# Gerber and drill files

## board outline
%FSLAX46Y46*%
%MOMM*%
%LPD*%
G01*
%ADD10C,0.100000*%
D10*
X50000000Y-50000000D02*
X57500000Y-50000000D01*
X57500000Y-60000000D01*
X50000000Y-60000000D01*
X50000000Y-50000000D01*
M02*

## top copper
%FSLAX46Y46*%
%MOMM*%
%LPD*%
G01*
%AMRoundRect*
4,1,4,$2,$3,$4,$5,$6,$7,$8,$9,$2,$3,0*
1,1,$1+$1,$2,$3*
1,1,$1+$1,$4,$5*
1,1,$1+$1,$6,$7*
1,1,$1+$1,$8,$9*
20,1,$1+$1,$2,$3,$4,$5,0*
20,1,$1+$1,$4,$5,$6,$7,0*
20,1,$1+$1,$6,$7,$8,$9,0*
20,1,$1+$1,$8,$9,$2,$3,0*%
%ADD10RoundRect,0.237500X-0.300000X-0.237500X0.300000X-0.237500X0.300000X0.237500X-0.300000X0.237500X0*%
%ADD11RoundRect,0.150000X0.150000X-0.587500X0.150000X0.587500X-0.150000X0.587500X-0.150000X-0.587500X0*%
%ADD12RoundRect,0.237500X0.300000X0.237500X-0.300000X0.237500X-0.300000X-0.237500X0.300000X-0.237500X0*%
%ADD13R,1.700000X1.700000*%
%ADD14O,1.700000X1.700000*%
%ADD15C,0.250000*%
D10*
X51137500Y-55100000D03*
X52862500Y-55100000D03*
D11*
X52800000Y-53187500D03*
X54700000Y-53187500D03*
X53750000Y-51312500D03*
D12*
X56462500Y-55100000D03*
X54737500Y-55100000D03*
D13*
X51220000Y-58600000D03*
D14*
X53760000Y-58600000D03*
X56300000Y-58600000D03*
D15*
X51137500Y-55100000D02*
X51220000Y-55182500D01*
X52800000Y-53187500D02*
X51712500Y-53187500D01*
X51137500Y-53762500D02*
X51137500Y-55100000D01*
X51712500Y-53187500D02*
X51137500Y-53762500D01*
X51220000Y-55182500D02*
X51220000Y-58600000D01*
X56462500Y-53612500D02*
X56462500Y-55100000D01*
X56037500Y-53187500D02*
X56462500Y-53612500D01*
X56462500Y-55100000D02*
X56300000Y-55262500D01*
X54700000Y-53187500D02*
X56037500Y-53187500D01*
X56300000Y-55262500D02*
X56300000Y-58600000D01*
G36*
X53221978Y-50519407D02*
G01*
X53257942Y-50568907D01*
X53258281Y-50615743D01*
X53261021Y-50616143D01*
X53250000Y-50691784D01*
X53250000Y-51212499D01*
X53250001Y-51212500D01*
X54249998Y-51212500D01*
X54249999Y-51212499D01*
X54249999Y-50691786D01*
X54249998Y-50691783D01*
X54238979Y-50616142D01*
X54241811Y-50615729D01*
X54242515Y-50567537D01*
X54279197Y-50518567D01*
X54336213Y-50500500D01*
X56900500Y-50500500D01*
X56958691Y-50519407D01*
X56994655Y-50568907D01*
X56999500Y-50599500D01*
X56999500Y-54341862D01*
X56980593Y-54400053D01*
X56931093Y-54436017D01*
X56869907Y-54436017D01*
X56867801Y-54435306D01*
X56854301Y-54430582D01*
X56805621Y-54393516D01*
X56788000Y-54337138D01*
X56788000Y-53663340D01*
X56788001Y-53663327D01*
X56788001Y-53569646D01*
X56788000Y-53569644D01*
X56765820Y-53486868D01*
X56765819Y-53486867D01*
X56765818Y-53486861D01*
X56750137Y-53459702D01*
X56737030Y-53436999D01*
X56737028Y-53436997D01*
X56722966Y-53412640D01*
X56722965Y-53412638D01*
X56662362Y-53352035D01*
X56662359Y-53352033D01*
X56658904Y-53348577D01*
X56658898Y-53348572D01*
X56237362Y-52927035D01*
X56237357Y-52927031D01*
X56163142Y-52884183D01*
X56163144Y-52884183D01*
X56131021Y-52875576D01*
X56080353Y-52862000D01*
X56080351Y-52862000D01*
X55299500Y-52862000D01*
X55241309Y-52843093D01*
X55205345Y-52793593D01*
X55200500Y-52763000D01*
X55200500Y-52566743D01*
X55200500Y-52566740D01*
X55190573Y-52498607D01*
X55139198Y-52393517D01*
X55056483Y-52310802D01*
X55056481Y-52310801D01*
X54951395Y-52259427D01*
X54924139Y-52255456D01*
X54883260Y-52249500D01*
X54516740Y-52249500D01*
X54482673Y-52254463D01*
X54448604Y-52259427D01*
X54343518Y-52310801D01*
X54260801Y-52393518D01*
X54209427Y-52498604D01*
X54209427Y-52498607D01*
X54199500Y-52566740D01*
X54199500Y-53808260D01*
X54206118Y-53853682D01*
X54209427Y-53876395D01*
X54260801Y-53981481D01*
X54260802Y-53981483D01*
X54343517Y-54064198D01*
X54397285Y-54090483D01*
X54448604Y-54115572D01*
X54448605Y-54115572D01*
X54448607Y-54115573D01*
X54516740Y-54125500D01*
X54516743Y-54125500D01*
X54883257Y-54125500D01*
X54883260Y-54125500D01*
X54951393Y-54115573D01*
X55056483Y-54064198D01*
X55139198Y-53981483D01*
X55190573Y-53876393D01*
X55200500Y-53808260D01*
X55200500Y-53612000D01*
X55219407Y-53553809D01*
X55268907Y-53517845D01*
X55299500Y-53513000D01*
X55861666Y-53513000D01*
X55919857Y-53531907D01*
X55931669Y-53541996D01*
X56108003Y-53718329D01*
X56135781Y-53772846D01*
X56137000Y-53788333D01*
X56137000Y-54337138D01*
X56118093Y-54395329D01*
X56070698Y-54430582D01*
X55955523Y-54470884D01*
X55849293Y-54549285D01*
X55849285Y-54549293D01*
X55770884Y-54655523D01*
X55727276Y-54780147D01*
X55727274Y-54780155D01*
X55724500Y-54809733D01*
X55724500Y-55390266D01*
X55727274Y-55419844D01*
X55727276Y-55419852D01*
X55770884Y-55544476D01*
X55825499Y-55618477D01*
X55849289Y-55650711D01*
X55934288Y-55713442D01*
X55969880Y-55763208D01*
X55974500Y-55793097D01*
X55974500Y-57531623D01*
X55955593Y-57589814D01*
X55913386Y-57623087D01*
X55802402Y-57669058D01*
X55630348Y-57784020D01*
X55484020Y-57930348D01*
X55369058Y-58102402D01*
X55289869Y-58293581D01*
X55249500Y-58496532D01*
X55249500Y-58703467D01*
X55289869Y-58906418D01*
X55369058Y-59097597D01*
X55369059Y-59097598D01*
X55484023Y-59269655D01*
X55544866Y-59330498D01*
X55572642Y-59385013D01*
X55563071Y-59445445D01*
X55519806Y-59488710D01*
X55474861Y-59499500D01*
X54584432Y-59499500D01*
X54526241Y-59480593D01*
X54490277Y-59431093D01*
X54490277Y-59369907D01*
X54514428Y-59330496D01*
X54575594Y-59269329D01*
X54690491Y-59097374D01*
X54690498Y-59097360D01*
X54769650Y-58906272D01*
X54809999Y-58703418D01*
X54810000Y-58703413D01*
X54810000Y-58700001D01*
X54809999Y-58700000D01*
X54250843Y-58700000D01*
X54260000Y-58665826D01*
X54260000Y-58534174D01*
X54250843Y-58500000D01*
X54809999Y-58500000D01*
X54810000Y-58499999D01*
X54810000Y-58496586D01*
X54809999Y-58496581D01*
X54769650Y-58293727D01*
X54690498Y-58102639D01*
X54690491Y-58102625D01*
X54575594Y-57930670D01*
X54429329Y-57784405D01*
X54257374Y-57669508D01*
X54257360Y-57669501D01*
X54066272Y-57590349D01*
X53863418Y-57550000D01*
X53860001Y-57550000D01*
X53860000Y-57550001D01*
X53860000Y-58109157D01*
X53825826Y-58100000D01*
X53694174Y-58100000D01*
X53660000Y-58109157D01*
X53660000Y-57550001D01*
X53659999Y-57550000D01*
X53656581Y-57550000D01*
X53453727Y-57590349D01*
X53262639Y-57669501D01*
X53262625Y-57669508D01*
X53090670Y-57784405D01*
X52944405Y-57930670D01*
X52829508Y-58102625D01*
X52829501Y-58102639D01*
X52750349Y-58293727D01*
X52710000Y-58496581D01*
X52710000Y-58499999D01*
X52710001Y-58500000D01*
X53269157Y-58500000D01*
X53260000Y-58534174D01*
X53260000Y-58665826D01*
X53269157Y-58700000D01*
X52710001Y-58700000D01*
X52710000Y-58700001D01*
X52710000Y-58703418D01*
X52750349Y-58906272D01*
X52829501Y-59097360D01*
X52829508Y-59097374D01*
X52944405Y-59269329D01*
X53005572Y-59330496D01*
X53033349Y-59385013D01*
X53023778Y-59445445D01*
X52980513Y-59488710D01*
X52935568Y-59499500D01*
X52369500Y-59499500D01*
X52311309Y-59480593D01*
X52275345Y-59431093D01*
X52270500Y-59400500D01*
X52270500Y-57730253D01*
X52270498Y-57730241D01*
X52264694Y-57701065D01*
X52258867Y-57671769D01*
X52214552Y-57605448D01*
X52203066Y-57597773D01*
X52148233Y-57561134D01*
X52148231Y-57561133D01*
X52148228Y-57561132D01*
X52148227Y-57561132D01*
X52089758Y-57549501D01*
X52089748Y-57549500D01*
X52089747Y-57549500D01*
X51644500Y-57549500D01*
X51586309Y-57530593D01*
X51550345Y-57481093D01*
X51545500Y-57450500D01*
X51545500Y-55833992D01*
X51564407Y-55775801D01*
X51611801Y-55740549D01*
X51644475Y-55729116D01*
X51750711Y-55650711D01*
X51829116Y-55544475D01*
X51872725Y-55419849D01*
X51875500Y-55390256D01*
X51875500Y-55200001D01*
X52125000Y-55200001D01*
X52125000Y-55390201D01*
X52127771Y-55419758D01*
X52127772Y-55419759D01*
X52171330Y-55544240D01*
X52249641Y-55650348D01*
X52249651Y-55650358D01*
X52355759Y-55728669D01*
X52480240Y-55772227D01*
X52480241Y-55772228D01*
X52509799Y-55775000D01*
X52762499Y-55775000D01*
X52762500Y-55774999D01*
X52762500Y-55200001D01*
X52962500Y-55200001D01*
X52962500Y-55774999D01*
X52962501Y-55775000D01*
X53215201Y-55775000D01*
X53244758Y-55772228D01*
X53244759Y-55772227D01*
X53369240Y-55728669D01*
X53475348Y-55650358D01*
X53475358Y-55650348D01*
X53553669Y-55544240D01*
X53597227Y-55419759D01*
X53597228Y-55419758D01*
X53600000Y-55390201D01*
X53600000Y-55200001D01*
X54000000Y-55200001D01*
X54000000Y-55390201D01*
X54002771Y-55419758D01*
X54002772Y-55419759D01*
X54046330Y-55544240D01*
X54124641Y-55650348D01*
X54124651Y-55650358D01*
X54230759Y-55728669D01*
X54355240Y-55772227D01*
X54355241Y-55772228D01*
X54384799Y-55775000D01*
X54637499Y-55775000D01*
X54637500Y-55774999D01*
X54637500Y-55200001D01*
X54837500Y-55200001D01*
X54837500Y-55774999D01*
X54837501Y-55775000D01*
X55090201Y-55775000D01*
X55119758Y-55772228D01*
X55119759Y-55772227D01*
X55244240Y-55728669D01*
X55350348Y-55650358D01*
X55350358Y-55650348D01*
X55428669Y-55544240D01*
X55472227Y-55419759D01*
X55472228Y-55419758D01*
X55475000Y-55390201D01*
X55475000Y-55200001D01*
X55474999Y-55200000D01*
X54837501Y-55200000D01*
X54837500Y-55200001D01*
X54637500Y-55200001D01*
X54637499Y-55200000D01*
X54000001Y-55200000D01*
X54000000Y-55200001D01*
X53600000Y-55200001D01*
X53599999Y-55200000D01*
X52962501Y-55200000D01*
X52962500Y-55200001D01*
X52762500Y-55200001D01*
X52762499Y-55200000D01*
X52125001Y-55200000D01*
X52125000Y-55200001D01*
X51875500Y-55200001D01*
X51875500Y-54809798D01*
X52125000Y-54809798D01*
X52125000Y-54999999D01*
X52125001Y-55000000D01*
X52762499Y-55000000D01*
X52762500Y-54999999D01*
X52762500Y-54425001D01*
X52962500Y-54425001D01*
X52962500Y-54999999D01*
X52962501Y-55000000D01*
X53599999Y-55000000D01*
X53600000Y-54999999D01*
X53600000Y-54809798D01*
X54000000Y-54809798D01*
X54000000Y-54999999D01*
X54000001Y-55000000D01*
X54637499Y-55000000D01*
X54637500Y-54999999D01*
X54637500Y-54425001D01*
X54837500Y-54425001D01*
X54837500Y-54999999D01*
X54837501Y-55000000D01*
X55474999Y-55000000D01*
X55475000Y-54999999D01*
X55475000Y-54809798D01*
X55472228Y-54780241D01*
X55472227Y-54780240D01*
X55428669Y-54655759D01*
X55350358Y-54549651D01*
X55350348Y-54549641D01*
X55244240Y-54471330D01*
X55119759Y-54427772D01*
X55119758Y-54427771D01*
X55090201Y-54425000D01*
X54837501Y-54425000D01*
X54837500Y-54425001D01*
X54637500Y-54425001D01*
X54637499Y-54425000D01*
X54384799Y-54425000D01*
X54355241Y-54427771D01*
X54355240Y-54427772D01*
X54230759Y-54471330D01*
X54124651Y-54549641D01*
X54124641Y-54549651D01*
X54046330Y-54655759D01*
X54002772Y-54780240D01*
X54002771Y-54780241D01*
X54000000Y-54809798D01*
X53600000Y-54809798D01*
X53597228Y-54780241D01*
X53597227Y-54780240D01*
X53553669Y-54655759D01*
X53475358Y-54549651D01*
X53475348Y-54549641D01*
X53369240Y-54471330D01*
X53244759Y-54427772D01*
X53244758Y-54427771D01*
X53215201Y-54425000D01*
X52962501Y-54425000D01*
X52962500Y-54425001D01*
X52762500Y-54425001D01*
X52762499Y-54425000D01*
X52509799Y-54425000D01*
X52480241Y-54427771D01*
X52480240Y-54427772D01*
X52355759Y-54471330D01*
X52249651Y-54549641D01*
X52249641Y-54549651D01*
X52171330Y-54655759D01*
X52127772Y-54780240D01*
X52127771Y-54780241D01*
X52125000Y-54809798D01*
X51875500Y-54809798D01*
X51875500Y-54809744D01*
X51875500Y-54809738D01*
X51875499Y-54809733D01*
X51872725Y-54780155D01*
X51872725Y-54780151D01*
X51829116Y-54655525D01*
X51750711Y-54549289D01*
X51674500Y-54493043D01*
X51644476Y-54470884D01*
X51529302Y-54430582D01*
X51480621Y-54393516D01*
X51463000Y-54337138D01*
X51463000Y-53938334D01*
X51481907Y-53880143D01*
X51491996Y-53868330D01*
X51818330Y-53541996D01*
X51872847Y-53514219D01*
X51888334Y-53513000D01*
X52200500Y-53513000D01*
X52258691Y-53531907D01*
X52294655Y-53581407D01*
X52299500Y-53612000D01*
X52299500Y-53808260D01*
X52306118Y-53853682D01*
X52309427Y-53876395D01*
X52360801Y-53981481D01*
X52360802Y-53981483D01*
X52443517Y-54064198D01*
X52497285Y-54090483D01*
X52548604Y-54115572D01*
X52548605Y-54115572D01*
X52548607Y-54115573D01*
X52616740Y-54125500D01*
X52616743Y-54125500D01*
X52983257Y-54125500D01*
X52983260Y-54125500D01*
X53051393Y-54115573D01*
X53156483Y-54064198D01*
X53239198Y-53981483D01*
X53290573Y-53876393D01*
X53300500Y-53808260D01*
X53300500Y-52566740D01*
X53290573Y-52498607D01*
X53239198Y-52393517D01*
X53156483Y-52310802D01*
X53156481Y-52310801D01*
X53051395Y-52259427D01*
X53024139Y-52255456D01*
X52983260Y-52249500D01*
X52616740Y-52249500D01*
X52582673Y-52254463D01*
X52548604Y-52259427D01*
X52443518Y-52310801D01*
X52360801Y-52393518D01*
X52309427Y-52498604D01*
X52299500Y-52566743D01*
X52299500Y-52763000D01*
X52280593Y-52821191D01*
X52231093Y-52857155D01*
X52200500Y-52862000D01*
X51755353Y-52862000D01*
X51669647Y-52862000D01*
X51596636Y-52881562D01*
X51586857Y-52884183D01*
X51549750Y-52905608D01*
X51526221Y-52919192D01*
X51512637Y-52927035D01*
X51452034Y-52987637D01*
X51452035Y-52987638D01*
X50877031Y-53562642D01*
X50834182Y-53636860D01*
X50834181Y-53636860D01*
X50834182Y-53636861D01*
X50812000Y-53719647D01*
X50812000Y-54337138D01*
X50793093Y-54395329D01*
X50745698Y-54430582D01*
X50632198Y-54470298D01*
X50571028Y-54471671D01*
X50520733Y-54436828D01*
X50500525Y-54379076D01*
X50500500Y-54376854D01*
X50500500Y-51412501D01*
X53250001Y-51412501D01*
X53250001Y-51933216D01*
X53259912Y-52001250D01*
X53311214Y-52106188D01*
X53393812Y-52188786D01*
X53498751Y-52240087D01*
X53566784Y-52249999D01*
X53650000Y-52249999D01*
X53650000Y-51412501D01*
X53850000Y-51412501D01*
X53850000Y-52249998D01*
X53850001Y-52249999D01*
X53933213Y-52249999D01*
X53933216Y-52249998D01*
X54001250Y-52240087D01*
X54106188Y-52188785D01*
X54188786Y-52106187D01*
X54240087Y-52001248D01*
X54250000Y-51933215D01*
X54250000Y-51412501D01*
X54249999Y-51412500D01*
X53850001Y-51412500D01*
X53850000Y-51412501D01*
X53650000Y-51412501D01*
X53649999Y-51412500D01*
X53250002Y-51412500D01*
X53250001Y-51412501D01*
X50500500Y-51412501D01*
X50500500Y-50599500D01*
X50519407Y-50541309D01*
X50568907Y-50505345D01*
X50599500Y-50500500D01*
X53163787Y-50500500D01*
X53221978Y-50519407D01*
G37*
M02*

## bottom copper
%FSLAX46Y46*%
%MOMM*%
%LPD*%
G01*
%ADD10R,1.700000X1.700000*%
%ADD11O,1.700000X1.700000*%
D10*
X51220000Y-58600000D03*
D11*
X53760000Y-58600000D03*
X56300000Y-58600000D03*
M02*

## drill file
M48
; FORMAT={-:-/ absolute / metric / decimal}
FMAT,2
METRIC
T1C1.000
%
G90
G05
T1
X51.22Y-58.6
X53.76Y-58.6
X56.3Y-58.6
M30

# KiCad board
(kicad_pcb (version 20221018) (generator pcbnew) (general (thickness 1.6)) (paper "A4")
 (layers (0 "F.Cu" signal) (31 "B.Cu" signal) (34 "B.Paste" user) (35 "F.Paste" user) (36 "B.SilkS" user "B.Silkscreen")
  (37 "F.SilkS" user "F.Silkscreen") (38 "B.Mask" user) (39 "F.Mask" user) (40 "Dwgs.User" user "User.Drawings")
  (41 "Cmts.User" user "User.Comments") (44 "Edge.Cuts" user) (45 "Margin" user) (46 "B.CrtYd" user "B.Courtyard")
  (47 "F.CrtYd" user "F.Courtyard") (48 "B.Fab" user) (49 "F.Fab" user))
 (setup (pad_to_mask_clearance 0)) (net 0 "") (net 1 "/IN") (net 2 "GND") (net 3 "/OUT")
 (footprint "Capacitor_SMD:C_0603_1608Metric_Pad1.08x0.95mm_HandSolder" (layer "F.Cu") (at 52 55.1)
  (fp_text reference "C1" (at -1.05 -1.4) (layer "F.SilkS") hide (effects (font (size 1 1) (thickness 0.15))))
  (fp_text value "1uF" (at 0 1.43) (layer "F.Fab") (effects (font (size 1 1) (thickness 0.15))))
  (pad "1" smd roundrect (at -0.8625 0) (size 1.075 0.95) (layers "F.Cu" "F.Paste" "F.Mask") (roundrect_rratio 0.25) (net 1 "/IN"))
  (pad "2" smd roundrect (at 0.8625 0) (size 1.075 0.95) (layers "F.Cu" "F.Paste" "F.Mask") (roundrect_rratio 0.25) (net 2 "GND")))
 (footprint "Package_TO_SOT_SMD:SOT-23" (layer "F.Cu") (at 53.75 52.25 90)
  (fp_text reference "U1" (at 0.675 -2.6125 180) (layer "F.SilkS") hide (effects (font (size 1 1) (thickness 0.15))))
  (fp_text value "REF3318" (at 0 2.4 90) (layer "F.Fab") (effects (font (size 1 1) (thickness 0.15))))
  (pad "1" smd roundrect (at -0.9375 -0.95 90) (size 1.475 0.6) (layers "F.Cu" "F.Paste" "F.Mask") (roundrect_rratio 0.25) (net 1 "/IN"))
  (pad "2" smd roundrect (at -0.9375 0.95 90) (size 1.475 0.6) (layers "F.Cu" "F.Paste" "F.Mask") (roundrect_rratio 0.25) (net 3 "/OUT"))
  (pad "3" smd roundrect (at 0.9375 0 90) (size 1.475 0.6) (layers "F.Cu" "F.Paste" "F.Mask") (roundrect_rratio 0.25) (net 2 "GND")))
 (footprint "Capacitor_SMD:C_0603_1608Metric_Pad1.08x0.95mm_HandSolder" (layer "F.Cu") (at 55.6 55.1 180)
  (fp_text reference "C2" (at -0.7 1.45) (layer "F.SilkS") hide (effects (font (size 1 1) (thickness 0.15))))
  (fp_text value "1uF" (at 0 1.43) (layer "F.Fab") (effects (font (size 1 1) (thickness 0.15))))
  (pad "1" smd roundrect (at -0.8625 0 180) (size 1.075 0.95) (layers "F.Cu" "F.Paste" "F.Mask") (roundrect_rratio 0.25) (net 3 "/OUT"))
  (pad "2" smd roundrect (at 0.8625 0 180) (size 1.075 0.95) (layers "F.Cu" "F.Paste" "F.Mask") (roundrect_rratio 0.25) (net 2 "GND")))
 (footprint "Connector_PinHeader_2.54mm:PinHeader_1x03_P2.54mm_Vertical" (layer "B.Cu") (at 51.22 58.6 -90)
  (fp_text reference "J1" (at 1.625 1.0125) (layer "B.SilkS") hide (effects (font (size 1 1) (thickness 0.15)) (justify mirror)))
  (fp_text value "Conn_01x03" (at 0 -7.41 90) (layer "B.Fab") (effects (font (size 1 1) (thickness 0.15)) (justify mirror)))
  (pad "1" thru_hole rect (at 0 0 270) (size 1.7 1.7) (drill 1) (layers "*.Cu" "*.Mask") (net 1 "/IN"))
  (pad "2" thru_hole oval (at 0 -2.54 270) (size 1.7 1.7) (drill 1) (layers "*.Cu" "*.Mask") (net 2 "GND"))
  (pad "3" thru_hole oval (at 0 -5.08 270) (size 1.7 1.7) (drill 1) (layers "*.Cu" "*.Mask") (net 3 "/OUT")))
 (gr_rect (start 50 50) (end 57.5 60) (stroke (width 0.1) (type default)) (fill none) (layer "Edge.Cuts"))
 (segment (start 51.1375 55.1) (end 51.22 55.1825) (width 0.25) (layer "F.Cu") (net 1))
 (segment (start 52.8 53.1875) (end 51.7125 53.1875) (width 0.25) (layer "F.Cu") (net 1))
 (segment (start 51.1375 53.7625) (end 51.1375 55.1) (width 0.25) (layer "F.Cu") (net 1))
 (segment (start 51.7125 53.1875) (end 51.1375 53.7625) (width 0.25) (layer "F.Cu") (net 1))
 (segment (start 51.22 55.1825) (end 51.22 58.6) (width 0.25) (layer "F.Cu") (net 1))
 (segment (start 56.4625 53.6125) (end 56.4625 55.1) (width 0.25) (layer "F.Cu") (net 3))
 (segment (start 56.0375 53.1875) (end 56.4625 53.6125) (width 0.25) (layer "F.Cu") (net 3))
 (segment (start 56.4625 55.1) (end 56.3 55.2625) (width 0.25) (layer "F.Cu") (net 3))
 (segment (start 54.7 53.1875) (end 56.0375 53.1875) (width 0.25) (layer "F.Cu") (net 3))
 (segment (start 56.3 55.2625) (end 56.3 58.6) (width 0.25) (layer "F.Cu") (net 3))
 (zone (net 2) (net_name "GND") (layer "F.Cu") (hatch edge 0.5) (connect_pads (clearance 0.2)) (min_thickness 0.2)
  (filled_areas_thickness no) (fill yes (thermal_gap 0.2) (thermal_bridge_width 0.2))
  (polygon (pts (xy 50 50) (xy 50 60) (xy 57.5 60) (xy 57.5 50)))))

